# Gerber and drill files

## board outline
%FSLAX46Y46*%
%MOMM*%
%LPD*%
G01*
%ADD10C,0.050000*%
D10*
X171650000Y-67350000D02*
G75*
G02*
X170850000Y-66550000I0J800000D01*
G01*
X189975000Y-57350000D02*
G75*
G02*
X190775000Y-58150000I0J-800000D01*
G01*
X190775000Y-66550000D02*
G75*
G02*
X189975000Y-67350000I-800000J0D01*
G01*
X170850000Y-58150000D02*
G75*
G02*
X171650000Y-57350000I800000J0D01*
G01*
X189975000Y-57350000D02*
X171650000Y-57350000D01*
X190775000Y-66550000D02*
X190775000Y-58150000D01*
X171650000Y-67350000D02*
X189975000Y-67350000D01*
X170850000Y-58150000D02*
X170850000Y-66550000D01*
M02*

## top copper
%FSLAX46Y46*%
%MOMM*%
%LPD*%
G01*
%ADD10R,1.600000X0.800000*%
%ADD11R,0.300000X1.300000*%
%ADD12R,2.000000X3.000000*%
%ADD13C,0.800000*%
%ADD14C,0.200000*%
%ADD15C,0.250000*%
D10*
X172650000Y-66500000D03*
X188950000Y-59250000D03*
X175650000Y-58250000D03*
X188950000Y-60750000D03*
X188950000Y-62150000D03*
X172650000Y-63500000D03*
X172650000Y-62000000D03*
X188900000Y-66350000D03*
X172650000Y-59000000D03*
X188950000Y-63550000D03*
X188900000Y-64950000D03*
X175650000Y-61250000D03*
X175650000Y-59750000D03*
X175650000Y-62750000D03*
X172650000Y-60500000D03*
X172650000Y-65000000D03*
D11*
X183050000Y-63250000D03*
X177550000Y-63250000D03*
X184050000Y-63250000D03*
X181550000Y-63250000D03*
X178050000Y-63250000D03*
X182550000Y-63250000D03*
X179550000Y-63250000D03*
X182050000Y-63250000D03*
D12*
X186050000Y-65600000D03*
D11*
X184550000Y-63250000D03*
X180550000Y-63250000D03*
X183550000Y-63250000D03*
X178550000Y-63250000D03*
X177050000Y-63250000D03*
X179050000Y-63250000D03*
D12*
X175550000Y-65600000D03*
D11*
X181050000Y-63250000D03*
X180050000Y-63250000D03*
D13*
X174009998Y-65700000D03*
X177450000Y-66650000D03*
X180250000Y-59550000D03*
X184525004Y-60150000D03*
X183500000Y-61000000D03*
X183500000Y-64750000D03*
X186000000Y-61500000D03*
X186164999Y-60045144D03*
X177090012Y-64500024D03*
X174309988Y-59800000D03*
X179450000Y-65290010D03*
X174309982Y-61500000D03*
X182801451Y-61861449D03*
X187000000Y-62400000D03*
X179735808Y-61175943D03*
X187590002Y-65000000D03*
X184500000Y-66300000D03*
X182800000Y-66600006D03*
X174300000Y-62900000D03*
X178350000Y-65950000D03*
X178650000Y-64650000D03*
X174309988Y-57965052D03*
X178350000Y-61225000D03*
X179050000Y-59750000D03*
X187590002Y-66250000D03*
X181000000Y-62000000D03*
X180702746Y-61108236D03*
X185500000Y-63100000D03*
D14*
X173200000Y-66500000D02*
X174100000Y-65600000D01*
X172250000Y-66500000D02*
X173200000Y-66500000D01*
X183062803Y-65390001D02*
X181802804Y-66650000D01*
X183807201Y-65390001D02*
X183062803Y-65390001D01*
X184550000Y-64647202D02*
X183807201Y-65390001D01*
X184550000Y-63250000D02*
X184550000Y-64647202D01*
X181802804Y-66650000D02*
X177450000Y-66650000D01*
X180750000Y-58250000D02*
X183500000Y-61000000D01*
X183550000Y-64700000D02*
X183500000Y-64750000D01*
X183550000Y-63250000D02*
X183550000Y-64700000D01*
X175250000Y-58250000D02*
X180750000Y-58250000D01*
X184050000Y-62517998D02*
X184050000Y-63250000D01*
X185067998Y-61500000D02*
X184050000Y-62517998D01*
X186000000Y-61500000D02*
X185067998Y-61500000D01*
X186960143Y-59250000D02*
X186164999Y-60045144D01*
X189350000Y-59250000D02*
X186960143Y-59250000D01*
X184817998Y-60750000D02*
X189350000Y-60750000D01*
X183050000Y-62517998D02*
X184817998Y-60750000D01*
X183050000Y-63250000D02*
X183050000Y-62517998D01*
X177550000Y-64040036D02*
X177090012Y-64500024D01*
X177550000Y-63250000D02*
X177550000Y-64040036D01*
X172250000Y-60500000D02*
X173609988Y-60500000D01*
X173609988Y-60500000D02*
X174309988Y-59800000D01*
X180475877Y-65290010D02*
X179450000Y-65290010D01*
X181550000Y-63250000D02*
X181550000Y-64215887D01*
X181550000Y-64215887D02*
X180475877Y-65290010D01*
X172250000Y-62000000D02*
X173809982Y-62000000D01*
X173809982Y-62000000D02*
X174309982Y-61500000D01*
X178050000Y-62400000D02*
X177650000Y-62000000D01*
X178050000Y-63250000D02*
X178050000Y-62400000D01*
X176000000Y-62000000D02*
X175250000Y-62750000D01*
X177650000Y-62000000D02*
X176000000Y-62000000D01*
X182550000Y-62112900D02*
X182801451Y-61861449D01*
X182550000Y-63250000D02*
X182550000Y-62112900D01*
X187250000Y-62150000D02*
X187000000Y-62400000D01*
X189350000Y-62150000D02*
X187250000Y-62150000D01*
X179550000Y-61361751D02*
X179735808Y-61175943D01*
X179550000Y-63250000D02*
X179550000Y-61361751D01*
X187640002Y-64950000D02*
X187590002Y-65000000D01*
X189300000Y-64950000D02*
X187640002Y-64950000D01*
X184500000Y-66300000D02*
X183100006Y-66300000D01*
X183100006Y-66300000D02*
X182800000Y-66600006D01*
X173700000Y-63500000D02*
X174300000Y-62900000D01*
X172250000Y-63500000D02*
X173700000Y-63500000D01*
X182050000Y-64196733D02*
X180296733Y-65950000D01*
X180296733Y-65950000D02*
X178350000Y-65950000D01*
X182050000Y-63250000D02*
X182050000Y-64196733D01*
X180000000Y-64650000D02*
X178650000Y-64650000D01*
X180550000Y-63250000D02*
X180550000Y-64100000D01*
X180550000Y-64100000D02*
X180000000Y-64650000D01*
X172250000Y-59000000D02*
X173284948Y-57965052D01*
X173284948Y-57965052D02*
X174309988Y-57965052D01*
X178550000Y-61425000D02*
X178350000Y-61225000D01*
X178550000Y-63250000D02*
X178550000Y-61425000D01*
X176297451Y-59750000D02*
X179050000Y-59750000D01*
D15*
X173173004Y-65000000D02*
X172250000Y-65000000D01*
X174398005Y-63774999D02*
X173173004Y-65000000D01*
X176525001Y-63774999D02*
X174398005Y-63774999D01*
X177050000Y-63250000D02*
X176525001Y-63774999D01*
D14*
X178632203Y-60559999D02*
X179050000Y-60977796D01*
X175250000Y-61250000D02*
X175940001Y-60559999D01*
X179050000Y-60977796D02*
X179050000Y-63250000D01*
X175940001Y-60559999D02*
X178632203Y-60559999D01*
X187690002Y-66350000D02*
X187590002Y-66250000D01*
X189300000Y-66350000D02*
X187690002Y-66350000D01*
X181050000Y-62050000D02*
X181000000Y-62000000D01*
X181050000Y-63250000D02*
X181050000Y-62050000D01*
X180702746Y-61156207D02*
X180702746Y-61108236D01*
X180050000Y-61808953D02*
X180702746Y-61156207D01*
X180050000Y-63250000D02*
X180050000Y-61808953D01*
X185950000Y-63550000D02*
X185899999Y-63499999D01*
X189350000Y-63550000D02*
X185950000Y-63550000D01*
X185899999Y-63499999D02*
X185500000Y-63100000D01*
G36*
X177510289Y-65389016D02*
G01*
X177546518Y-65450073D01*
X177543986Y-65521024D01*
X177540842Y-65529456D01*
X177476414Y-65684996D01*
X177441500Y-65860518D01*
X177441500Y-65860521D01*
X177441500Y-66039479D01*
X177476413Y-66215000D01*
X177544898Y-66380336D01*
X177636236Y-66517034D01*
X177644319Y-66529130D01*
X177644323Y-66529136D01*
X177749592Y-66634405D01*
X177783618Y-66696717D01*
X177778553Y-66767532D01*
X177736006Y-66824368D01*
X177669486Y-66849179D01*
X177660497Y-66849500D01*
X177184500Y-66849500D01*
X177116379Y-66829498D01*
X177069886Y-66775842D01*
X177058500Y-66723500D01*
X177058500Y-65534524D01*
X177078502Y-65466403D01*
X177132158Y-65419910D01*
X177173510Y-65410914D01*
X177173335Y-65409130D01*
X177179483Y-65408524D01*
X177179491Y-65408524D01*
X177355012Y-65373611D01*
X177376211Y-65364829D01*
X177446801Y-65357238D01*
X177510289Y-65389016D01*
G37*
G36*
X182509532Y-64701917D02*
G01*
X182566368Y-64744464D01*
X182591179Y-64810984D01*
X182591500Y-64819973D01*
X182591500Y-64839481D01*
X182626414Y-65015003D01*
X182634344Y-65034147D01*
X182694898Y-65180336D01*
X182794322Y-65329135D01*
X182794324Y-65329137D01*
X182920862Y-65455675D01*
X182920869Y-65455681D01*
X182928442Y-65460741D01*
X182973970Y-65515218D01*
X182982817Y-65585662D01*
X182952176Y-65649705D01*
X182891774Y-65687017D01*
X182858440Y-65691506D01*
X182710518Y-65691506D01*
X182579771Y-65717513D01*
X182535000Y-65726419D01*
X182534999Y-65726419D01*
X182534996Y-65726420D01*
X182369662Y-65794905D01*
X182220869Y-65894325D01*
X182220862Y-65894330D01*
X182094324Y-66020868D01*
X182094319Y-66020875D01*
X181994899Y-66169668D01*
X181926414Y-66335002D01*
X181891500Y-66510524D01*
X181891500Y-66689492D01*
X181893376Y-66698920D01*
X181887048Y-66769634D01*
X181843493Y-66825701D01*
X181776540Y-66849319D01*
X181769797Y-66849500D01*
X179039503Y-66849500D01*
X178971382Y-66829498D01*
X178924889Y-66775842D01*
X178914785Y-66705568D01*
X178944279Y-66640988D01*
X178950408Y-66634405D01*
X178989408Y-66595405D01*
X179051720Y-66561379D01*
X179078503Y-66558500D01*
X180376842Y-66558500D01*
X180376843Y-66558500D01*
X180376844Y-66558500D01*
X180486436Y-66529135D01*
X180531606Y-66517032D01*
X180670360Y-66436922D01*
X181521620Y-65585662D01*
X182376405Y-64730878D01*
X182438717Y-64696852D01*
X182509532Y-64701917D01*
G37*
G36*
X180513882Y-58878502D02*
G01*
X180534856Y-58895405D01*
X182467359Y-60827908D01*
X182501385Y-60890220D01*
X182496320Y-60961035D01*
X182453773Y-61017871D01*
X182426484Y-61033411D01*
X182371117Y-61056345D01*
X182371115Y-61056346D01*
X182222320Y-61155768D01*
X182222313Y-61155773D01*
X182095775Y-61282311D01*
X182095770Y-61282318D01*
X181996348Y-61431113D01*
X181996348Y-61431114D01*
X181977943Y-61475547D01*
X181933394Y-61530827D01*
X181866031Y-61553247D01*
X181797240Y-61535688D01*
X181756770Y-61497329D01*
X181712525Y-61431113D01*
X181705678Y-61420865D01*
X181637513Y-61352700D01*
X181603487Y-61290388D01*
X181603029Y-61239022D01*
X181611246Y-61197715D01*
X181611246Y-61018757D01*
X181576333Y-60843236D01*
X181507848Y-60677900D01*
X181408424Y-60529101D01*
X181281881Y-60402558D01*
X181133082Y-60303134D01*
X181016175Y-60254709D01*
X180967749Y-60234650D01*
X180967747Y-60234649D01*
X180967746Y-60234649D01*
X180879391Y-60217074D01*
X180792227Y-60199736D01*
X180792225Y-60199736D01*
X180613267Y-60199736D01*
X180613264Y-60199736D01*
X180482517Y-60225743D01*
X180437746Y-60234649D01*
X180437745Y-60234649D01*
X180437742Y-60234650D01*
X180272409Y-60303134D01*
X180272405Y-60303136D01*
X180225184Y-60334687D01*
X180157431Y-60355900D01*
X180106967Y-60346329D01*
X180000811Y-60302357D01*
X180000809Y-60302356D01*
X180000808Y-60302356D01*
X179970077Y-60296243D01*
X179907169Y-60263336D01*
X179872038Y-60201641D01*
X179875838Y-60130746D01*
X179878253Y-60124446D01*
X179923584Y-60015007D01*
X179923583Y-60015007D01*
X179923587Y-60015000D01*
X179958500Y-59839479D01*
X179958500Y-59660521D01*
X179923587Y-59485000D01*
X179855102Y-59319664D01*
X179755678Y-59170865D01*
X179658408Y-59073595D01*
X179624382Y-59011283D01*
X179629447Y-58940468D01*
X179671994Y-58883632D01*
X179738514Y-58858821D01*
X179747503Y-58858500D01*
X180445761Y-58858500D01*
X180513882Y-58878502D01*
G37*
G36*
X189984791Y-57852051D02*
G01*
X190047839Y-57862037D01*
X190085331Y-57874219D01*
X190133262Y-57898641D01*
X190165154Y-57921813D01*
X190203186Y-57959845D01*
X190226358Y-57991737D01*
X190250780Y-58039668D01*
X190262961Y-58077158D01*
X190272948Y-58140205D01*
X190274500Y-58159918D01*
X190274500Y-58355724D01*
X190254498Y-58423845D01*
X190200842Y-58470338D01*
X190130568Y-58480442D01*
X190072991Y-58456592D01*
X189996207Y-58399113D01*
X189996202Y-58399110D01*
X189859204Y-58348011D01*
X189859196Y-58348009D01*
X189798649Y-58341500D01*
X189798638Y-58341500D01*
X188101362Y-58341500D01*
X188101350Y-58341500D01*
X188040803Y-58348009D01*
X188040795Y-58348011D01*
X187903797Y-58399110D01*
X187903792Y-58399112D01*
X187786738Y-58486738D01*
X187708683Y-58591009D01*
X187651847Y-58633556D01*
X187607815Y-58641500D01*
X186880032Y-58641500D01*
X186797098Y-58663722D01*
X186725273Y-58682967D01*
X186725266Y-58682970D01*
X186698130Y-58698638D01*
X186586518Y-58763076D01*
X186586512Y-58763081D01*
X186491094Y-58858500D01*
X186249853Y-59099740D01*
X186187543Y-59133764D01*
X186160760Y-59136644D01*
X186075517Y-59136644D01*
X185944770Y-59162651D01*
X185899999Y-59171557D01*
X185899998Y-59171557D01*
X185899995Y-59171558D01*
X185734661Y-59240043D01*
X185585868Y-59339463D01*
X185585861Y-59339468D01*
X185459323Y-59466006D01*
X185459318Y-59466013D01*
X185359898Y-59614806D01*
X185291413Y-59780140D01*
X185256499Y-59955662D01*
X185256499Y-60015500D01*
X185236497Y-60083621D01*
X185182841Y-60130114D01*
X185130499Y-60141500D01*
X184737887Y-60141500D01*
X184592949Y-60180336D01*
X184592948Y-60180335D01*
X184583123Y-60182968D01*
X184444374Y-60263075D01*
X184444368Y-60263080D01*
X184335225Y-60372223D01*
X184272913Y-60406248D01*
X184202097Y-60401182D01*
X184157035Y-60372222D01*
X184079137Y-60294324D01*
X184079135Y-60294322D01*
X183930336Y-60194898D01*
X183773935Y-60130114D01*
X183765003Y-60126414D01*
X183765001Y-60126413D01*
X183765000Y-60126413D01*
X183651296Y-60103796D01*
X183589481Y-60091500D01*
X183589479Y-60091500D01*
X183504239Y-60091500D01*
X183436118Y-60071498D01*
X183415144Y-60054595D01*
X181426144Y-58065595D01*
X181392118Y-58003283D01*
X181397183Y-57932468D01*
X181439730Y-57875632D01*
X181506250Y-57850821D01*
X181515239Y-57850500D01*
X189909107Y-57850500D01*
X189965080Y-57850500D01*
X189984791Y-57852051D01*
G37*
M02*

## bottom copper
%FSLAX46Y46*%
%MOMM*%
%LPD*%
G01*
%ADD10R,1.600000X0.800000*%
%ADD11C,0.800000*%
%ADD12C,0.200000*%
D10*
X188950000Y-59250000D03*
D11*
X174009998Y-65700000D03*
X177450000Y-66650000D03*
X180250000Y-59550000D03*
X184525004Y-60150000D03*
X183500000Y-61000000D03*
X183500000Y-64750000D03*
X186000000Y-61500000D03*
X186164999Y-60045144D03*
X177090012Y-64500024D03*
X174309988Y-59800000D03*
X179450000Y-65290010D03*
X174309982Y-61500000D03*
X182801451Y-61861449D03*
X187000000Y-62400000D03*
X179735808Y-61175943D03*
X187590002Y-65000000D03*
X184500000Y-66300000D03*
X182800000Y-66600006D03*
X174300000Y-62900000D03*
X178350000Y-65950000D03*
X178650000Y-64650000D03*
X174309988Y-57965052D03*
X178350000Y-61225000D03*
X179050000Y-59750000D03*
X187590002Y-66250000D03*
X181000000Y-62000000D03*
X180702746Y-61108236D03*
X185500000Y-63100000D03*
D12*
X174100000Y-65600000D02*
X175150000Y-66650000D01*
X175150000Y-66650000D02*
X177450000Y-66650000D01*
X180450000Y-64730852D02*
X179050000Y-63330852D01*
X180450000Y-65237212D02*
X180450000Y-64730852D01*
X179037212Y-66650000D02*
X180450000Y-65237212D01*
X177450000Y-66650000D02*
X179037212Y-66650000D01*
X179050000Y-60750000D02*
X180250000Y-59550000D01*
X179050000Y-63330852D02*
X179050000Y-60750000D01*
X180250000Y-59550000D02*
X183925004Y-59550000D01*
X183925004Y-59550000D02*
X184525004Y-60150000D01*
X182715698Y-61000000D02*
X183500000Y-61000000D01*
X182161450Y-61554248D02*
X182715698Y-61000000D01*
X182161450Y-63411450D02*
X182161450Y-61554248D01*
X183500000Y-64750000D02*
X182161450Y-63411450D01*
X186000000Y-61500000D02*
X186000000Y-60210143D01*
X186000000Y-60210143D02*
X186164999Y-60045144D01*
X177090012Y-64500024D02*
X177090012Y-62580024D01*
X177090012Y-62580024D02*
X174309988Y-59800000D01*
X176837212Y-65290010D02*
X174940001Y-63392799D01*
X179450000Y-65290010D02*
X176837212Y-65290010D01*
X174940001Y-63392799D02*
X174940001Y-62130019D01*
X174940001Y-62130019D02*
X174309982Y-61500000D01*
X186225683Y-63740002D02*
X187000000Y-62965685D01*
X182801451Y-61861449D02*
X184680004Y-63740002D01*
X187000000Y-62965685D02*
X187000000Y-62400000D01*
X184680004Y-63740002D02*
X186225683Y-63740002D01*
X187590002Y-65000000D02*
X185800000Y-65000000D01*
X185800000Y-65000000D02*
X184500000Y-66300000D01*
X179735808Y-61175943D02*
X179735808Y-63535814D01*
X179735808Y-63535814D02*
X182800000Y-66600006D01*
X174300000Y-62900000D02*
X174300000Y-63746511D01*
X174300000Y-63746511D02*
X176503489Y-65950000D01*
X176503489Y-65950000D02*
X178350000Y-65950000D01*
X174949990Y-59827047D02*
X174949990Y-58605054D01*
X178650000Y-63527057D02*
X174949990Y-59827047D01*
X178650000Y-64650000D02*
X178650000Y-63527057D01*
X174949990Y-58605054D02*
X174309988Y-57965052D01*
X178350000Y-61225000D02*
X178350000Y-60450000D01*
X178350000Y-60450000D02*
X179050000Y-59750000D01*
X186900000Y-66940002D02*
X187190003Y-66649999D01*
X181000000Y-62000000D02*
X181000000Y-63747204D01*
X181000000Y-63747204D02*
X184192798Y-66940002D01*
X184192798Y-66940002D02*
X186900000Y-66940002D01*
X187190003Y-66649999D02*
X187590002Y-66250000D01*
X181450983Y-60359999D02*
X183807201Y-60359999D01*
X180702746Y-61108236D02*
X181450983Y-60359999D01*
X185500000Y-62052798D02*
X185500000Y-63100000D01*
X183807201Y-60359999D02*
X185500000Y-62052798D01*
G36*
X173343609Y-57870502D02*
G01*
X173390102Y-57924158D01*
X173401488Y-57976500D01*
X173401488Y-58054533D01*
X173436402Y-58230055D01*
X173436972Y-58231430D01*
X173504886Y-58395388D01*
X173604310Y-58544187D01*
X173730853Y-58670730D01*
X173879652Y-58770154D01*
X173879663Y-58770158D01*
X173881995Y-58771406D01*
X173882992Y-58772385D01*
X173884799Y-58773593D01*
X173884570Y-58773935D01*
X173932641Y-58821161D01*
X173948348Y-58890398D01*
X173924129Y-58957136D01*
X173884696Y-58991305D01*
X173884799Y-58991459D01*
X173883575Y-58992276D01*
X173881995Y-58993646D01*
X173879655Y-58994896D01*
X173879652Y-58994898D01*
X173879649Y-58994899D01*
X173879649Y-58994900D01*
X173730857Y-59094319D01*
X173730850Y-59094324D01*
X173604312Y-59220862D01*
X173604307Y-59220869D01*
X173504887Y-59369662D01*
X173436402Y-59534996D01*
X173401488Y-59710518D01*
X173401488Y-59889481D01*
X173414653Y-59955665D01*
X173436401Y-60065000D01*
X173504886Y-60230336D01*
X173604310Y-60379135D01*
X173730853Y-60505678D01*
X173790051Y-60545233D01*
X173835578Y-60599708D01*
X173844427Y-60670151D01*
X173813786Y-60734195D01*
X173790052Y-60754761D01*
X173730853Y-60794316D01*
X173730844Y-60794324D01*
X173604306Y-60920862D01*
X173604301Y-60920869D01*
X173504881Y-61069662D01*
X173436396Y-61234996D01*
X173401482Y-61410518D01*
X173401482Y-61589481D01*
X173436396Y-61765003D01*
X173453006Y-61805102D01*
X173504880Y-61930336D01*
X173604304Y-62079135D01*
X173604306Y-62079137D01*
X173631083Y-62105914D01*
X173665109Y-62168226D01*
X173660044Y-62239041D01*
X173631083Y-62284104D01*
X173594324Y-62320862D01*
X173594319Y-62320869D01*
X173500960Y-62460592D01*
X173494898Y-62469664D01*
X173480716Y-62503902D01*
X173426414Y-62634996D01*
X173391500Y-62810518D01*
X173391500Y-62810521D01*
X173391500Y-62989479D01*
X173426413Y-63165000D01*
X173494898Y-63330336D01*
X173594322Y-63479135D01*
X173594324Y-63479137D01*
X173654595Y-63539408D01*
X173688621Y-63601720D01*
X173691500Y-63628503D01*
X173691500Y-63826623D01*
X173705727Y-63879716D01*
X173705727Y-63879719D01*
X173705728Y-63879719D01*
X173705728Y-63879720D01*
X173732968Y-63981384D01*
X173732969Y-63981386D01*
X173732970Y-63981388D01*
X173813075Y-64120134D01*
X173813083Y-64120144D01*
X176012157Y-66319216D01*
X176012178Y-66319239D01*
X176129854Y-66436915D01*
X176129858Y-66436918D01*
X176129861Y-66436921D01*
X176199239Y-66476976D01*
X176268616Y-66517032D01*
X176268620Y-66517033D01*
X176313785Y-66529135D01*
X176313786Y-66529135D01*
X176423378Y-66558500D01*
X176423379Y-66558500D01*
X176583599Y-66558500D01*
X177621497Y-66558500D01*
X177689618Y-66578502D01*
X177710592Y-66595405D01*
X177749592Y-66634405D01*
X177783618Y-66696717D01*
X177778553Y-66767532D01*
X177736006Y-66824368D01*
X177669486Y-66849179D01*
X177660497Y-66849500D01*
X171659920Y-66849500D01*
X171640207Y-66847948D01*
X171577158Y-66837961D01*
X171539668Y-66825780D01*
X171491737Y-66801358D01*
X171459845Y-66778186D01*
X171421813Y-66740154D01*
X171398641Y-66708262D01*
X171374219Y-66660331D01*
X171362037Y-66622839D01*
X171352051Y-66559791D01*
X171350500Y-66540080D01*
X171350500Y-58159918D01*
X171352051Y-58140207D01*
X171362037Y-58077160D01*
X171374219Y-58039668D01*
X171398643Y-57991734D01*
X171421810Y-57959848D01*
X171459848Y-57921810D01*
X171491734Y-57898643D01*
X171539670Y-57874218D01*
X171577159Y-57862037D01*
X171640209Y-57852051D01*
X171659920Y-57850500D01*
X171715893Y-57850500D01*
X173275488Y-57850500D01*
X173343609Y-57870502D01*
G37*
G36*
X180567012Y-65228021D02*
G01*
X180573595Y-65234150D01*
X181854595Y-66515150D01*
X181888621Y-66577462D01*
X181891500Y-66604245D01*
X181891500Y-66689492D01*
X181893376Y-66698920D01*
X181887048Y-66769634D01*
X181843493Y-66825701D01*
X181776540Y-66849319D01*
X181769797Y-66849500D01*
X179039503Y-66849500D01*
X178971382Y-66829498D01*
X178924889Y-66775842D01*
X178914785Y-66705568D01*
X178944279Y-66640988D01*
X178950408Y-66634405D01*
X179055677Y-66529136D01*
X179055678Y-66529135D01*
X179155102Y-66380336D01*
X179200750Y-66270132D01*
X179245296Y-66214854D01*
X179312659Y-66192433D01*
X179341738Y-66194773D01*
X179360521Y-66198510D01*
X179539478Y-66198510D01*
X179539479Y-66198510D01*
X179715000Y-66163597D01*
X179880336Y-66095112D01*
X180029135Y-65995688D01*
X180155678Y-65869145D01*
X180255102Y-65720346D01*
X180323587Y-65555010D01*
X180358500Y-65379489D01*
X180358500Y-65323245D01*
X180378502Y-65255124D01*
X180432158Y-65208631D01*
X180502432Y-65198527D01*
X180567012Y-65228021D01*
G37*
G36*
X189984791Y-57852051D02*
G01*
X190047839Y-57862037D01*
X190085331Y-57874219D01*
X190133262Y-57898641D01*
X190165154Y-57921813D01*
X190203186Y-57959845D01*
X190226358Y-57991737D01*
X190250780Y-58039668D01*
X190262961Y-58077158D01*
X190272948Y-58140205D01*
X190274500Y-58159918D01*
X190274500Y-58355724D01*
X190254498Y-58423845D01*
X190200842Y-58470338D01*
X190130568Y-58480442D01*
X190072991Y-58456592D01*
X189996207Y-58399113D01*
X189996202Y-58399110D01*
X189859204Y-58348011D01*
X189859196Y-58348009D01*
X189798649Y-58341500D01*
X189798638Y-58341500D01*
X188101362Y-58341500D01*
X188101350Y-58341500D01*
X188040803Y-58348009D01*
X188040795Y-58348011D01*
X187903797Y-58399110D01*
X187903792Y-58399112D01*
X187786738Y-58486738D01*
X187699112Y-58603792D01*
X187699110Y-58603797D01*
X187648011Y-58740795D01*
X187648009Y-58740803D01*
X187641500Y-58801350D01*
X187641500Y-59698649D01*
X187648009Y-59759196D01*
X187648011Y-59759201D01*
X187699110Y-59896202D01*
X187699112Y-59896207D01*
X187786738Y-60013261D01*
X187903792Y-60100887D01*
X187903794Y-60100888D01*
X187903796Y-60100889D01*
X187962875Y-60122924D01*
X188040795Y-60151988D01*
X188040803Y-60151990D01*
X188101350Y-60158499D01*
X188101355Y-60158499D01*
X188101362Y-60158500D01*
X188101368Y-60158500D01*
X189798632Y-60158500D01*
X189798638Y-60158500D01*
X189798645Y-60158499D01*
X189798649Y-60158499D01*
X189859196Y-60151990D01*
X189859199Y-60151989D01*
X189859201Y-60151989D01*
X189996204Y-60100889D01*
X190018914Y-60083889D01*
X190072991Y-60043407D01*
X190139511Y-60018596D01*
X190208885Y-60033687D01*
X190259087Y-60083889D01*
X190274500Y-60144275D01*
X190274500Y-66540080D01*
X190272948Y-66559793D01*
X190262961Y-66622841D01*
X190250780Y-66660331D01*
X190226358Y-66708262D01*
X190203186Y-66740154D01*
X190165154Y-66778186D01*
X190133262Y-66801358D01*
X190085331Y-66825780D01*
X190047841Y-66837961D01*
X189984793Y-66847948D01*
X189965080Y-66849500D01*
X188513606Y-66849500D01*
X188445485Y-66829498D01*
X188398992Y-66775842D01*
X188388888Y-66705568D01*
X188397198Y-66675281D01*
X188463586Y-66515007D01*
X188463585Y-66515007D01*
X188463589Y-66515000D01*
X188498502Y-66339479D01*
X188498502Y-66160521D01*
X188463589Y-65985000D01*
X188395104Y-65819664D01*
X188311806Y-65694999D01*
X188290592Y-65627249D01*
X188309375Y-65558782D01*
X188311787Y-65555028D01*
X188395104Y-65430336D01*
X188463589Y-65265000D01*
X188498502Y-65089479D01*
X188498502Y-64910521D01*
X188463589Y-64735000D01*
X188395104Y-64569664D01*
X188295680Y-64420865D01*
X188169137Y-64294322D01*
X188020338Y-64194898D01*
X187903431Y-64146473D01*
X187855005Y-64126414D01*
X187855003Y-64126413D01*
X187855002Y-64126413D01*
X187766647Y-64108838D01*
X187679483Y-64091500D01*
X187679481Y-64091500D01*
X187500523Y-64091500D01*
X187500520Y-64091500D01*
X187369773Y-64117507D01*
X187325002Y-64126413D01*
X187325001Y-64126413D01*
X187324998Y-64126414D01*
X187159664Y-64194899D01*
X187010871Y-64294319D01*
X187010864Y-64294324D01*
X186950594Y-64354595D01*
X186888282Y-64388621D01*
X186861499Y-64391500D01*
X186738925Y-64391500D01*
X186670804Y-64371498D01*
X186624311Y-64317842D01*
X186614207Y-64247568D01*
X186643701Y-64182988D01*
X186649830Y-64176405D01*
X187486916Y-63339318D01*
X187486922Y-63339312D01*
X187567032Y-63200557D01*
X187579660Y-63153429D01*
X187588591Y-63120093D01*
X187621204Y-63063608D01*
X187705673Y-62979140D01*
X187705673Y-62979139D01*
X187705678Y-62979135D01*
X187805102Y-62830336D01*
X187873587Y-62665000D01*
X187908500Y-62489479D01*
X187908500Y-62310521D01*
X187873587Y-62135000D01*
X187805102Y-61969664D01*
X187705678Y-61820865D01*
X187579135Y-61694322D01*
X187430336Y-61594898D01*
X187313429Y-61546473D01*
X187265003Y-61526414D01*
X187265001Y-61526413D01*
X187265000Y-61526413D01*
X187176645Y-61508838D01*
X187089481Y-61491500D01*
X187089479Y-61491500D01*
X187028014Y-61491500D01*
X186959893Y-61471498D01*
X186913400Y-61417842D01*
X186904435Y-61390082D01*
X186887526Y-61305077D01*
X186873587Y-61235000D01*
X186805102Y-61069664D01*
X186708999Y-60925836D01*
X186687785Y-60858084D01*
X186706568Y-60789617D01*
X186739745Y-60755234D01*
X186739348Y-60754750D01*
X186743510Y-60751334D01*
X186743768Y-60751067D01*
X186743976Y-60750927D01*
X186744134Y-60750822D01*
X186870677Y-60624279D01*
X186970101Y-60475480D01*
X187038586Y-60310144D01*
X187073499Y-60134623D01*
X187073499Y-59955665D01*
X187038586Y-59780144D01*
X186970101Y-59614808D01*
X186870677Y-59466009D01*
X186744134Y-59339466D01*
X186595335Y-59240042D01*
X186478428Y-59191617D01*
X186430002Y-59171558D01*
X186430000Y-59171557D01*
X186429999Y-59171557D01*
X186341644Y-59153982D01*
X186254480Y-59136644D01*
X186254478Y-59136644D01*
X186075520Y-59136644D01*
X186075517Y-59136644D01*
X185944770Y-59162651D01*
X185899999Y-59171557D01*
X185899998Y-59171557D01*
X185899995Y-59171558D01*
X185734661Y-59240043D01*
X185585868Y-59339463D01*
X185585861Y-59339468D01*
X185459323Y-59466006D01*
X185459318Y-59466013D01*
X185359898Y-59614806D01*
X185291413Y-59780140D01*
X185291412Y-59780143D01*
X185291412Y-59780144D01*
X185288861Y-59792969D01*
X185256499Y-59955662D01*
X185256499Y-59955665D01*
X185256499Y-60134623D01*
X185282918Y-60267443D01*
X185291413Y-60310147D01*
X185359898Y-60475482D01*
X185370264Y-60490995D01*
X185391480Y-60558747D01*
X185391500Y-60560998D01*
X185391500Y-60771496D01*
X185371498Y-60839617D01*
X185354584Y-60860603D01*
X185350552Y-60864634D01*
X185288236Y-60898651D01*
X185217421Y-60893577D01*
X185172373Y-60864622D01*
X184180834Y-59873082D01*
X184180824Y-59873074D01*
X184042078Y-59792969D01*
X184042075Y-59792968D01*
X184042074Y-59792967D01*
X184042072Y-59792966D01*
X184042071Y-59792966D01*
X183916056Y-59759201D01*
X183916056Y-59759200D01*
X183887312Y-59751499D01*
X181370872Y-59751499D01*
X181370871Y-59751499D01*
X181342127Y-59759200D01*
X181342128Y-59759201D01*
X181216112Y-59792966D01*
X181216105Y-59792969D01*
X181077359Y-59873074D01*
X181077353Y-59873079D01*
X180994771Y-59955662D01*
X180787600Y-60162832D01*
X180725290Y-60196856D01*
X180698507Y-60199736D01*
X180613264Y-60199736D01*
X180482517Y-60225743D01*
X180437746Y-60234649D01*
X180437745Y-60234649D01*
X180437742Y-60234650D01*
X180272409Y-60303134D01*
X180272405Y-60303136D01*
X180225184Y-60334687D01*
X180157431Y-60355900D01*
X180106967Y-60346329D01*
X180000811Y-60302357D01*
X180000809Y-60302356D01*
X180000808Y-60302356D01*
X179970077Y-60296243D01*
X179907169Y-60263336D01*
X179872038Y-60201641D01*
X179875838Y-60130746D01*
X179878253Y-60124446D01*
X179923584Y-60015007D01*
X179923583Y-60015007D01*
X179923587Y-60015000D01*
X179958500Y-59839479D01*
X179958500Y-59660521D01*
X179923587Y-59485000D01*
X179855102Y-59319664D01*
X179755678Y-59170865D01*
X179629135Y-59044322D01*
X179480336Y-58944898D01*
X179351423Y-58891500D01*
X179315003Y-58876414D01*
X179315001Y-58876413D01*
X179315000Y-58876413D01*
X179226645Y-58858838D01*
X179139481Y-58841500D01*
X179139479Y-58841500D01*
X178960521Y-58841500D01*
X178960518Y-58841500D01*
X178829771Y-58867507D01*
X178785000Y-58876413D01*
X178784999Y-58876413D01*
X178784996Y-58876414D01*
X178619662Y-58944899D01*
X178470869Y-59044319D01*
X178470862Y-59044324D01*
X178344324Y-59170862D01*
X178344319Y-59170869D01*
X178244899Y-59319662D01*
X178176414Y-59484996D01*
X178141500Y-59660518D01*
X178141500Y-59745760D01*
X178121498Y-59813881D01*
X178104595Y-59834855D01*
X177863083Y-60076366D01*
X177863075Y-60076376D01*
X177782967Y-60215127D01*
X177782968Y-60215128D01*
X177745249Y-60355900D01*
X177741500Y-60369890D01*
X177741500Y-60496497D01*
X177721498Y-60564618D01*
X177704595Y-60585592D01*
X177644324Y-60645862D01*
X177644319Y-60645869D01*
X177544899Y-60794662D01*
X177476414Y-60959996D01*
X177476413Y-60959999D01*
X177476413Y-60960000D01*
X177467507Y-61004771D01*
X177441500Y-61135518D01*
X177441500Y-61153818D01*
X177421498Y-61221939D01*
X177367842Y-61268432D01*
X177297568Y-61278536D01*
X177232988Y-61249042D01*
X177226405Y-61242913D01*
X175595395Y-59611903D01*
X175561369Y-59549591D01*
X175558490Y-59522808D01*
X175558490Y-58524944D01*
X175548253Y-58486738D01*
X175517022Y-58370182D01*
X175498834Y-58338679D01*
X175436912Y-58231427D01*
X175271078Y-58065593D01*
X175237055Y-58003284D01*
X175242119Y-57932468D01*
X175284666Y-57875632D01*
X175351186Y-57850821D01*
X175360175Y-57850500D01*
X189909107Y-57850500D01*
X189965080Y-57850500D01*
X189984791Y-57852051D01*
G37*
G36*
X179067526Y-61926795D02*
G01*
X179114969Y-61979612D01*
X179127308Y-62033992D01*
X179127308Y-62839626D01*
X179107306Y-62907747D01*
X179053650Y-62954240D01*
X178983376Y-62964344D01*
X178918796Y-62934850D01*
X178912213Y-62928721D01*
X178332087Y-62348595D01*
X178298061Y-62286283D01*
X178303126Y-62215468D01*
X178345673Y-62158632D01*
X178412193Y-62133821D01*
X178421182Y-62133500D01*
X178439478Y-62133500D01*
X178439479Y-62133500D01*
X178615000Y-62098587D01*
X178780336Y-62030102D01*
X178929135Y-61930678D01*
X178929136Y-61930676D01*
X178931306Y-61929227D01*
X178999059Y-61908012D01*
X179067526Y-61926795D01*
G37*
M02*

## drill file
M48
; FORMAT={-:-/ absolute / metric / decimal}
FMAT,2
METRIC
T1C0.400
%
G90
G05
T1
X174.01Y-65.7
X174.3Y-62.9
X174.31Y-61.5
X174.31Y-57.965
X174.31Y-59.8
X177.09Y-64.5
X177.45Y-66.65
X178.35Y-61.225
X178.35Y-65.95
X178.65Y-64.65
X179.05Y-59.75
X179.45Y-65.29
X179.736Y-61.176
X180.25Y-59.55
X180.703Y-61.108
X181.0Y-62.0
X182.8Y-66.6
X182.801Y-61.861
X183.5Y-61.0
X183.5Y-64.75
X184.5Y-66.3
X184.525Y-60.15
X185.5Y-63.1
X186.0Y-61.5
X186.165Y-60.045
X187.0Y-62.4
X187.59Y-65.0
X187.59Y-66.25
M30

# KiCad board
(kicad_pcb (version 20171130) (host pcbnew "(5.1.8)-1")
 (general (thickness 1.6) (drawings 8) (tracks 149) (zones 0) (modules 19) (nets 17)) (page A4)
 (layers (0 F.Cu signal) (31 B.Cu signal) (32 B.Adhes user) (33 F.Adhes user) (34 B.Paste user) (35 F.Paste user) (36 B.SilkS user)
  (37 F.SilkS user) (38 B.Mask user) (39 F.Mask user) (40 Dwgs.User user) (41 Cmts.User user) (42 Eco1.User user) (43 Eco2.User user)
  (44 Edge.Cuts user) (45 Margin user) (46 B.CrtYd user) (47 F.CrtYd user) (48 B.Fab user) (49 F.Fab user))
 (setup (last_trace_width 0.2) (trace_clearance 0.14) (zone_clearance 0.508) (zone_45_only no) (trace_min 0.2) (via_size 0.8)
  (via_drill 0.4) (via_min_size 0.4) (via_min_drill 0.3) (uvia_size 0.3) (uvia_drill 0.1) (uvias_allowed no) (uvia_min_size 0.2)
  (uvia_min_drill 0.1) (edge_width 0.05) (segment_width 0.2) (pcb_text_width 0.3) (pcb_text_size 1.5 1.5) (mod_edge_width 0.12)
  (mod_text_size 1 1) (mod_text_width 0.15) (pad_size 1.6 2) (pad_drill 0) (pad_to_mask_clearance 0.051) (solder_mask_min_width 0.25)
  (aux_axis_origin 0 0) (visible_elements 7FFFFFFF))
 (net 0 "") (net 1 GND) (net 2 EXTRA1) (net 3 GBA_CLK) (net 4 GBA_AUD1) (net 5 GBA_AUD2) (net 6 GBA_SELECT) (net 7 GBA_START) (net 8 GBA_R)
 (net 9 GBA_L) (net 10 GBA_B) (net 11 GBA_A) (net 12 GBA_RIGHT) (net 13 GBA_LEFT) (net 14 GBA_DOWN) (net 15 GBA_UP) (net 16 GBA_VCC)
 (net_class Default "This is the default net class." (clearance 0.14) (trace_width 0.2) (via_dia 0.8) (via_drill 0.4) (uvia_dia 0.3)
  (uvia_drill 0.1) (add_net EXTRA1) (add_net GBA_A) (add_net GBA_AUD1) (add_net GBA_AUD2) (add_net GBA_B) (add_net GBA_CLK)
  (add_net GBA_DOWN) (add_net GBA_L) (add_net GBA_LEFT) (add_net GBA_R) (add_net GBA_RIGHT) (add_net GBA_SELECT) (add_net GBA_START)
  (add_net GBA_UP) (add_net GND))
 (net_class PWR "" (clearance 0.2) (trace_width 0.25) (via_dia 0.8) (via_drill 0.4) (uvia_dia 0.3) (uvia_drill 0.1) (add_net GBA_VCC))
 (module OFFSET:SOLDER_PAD (layer B.Cu) (at 188.8 59.25 270)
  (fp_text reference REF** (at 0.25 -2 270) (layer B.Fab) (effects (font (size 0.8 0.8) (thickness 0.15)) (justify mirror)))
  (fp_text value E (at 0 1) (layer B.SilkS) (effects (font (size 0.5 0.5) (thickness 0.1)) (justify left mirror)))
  (pad 1 smd rect (at 0 0.25 270) (size 0.8 1.6) (drill (offset 0 -0.4)) (layers B.Cu B.Paste B.Mask)))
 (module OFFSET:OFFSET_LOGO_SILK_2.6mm (layer B.Cu) (at 180.575 62.275 180)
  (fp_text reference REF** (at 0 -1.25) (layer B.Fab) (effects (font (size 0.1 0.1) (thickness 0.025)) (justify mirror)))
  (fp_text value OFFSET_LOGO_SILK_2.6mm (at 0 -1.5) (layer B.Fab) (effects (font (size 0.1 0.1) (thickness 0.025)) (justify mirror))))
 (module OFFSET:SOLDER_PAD (layer F.Cu) (at 172.5 66.5 90)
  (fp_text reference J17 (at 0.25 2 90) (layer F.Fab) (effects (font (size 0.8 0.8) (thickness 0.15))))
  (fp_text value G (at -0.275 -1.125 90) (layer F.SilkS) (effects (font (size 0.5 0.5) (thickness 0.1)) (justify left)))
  (pad 1 smd rect (at 0 -0.25 90) (size 0.8 1.6) (drill (offset 0 0.4)) (layers F.Cu F.Paste F.Mask) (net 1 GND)))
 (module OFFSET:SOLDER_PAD (layer F.Cu) (at 189.1 59.25 270)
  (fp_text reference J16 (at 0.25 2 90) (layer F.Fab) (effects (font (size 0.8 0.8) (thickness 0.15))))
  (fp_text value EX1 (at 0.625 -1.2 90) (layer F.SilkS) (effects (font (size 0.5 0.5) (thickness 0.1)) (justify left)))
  (pad 1 smd rect (at 0 -0.25 270) (size 0.8 1.6) (drill (offset 0 0.4)) (layers F.Cu F.Paste F.Mask) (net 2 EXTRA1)))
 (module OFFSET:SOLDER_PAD (layer F.Cu) (at 175.5 58.25 90)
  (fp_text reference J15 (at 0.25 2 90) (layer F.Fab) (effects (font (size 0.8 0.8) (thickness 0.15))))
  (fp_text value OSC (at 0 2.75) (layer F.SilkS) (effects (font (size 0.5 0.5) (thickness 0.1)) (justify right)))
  (pad 1 smd rect (at 0 -0.25 90) (size 0.8 1.6) (drill (offset 0 0.4)) (layers F.Cu F.Paste F.Mask) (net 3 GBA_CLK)))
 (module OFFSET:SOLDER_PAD (layer F.Cu) (at 189.1 60.75 270)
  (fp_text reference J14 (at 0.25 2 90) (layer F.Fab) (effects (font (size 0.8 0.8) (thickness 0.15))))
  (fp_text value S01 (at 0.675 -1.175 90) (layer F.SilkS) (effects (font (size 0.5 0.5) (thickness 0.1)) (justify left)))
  (pad 1 smd rect (at 0 -0.25 270) (size 0.8 1.6) (drill (offset 0 0.4)) (layers F.Cu F.Paste F.Mask) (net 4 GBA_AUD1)))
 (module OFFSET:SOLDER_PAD (layer F.Cu) (at 189.1 62.15 270)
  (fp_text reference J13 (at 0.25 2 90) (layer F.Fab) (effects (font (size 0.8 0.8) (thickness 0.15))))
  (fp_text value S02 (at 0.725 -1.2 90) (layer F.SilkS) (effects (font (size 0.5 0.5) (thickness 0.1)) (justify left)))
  (pad 1 smd rect (at 0 -0.25 270) (size 0.8 1.6) (drill (offset 0 0.4)) (layers F.Cu F.Paste F.Mask) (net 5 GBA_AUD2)))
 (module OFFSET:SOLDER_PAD (layer F.Cu) (at 172.5 63.5 90)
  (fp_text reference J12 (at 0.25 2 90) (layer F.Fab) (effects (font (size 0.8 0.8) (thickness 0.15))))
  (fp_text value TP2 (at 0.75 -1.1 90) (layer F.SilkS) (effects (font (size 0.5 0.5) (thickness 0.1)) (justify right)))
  (pad 1 smd rect (at 0 -0.25 90) (size 0.8 1.6) (drill (offset 0 0.4)) (layers F.Cu F.Paste F.Mask) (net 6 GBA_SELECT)))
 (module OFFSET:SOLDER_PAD (layer F.Cu) (at 172.5 62 90)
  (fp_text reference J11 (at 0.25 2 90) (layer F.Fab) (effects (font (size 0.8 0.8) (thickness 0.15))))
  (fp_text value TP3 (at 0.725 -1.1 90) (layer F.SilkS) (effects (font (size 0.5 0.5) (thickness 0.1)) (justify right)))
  (pad 1 smd rect (at 0 -0.25 90) (size 0.8 1.6) (drill (offset 0 0.4)) (layers F.Cu F.Paste F.Mask) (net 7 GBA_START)))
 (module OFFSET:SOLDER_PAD (layer F.Cu) (at 189.05 66.35 270)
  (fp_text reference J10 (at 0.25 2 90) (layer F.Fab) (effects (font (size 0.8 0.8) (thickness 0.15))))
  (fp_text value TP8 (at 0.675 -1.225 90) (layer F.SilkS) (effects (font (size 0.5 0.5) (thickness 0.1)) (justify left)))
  (pad 1 smd rect (at 0 -0.25 270) (size 0.8 1.6) (drill (offset 0 0.4)) (layers F.Cu F.Paste F.Mask) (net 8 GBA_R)))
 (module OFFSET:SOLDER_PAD (layer F.Cu) (at 172.5 59 90)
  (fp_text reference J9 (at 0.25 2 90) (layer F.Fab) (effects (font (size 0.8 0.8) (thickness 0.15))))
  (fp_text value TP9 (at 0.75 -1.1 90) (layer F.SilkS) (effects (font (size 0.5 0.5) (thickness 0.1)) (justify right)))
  (pad 1 smd rect (at 0 -0.25 90) (size 0.8 1.6) (drill (offset 0 0.4)) (layers F.Cu F.Paste F.Mask) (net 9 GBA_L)))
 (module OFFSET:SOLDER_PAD (layer F.Cu) (at 189.1 63.55 270)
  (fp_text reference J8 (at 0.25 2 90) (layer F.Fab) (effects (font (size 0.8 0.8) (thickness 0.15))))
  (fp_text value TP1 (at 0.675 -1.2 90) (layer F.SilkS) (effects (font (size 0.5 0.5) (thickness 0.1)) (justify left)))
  (pad 1 smd rect (at 0 -0.25 270) (size 0.8 1.6) (drill (offset 0 0.4)) (layers F.Cu F.Paste F.Mask) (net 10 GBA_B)))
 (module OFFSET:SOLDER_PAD (layer F.Cu) (at 189.05 64.95 270)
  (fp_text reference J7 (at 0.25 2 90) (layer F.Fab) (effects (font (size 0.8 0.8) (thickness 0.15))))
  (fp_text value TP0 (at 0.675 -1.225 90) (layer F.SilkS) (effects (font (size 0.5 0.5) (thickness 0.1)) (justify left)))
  (pad 1 smd rect (at 0 -0.25 270) (size 0.8 1.6) (drill (offset 0 0.4)) (layers F.Cu F.Paste F.Mask) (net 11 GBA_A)))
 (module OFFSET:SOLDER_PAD (layer F.Cu) (at 175.5 61.25 90)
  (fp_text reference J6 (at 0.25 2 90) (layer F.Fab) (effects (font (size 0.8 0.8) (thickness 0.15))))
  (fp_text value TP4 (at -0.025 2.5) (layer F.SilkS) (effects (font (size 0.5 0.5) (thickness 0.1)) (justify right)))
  (pad 1 smd rect (at 0 -0.25 90) (size 0.8 1.6) (drill (offset 0 0.4)) (layers F.Cu F.Paste F.Mask) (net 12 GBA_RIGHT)))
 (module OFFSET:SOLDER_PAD (layer F.Cu) (at 175.5 59.75 90)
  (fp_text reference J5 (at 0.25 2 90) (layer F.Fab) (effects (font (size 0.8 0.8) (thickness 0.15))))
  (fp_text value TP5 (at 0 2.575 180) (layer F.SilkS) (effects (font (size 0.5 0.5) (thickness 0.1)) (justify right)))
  (pad 1 smd rect (at 0 -0.25 90) (size 0.8 1.6) (drill (offset 0 0.4)) (layers F.Cu F.Paste F.Mask) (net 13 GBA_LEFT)))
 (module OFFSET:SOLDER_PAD (layer F.Cu) (at 175.5 62.75 90)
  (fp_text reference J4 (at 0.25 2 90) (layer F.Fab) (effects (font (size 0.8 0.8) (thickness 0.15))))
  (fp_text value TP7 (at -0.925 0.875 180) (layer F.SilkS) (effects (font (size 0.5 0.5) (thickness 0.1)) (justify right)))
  (pad 1 smd rect (at 0 -0.25 90) (size 0.8 1.6) (drill (offset 0 0.4)) (layers F.Cu F.Paste F.Mask) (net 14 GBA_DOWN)))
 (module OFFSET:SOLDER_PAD (layer F.Cu) (at 172.5 60.5 90)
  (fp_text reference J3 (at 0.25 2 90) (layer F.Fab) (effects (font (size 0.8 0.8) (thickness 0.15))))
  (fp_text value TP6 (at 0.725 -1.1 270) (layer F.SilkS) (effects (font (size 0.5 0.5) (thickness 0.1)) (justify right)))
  (pad 1 smd rect (at 0 -0.25 90) (size 0.8 1.6) (drill (offset 0 0.4)) (layers F.Cu F.Paste F.Mask) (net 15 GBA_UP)))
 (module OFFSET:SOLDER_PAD (layer F.Cu) (at 172.5 65 90)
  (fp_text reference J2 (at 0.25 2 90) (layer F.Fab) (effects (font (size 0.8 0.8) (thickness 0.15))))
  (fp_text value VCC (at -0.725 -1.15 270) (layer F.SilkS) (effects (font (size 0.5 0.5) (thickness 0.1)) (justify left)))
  (pad 1 smd rect (at 0 -0.25 90) (size 0.8 1.6) (drill (offset 0 0.4)) (layers F.Cu F.Paste F.Mask) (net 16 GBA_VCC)))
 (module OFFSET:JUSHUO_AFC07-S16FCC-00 (layer F.Cu) (at 180.8 65)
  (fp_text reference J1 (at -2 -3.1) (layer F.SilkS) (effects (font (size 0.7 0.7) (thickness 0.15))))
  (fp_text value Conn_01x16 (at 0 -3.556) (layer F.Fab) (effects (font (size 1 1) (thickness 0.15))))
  (pad 13 smd rect (at 2.25 -1.75) (size 0.3 1.3) (layers F.Cu F.Paste F.Mask) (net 4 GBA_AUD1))
  (pad 2 smd rect (at -3.25 -1.75) (size 0.3 1.3) (layers F.Cu F.Paste F.Mask) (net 15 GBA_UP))
  (pad 15 smd rect (at 3.25 -1.75) (size 0.3 1.3) (layers F.Cu F.Paste F.Mask) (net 2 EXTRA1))
  (pad 10 smd rect (at 0.75 -1.75) (size 0.3 1.3) (layers F.Cu F.Paste F.Mask) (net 7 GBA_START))
  (pad 3 smd rect (at -2.75 -1.75) (size 0.3 1.3) (layers F.Cu F.Paste F.Mask) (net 14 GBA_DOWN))
  (pad 12 smd rect (at 1.75 -1.75) (size 0.3 1.3) (layers F.Cu F.Paste F.Mask) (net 5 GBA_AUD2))
  (pad 6 smd rect (at -1.25 -1.75) (size 0.3 1.3) (layers F.Cu F.Paste F.Mask) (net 11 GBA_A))
  (pad 11 smd rect (at 1.25 -1.75) (size 0.3 1.3) (layers F.Cu F.Paste F.Mask) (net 6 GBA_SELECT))
  (pad "" smd rect (at 5.25 0.6) (size 2 3) (layers F.Cu F.Paste F.Mask))
  (pad 16 smd rect (at 3.75 -1.75) (size 0.3 1.3) (layers F.Cu F.Paste F.Mask) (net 1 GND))
  (pad 8 smd rect (at -0.25 -1.75) (size 0.3 1.3) (layers F.Cu F.Paste F.Mask) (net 9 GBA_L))
  (pad 14 smd rect (at 2.75 -1.75) (size 0.3 1.3) (layers F.Cu F.Paste F.Mask) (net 3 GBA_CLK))
  (pad 4 smd rect (at -2.25 -1.75) (size 0.3 1.3) (layers F.Cu F.Paste F.Mask) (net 13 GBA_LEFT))
  (pad 1 smd rect (at -3.75 -1.75) (size 0.3 1.3) (layers F.Cu F.Paste F.Mask) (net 16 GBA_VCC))
  (pad 5 smd rect (at -1.75 -1.75) (size 0.3 1.3) (layers F.Cu F.Paste F.Mask) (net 12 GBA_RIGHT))
  (pad "" smd rect (at -5.25 0.6) (size 2 3) (layers F.Cu F.Paste F.Mask))
  (pad 9 smd rect (at 0.25 -1.75) (size 0.3 1.3) (layers F.Cu F.Paste F.Mask) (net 8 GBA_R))
  (pad 7 smd rect (at -0.75 -1.75) (size 0.3 1.3) (layers F.Cu F.Paste F.Mask) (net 10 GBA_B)))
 (gr_arc (start 171.65 66.55) (end 171.65 67.35) (angle 90) (layer Edge.Cuts) (width 0.05))
 (gr_arc (start 189.975 58.15) (end 190.775 58.15) (angle -90) (layer Edge.Cuts) (width 0.05))
 (gr_arc (start 189.975 66.55) (end 189.975 67.35) (angle -90) (layer Edge.Cuts) (width 0.05))
 (gr_arc (start 171.65 58.15) (end 171.65 57.35) (angle -90) (layer Edge.Cuts) (width 0.05))
 (gr_line (start 189.975 57.35) (end 171.65 57.35) (layer Edge.Cuts) (width 0.05))
 (gr_line (start 190.775 66.55) (end 190.775 58.15) (layer Edge.Cuts) (width 0.05))
 (gr_line (start 171.65 67.35) (end 189.975 67.35) (layer Edge.Cuts) (width 0.05))
 (gr_line (start 170.85 58.15) (end 170.85 66.55) (layer Edge.Cuts) (width 0.05))
 (via (at 174.009998 65.7) (size 0.8) (drill 0.4) (layers F.Cu B.Cu) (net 1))
 (segment (start 173.2 66.5) (end 174.1 65.6) (width 0.2) (layer F.Cu) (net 1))
 (segment (start 172.25 66.5) (end 173.2 66.5) (width 0.2) (layer F.Cu) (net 1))
 (segment (start 183.062803 65.390001) (end 181.802804 66.65) (width 0.2) (layer F.Cu) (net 1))
 (segment (start 183.807201 65.390001) (end 183.062803 65.390001) (width 0.2) (layer F.Cu) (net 1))
 (segment (start 184.55 64.647202) (end 183.807201 65.390001) (width 0.2) (layer F.Cu) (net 1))
 (segment (start 184.55 63.25) (end 184.55 64.647202) (width 0.2) (layer F.Cu) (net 1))
 (segment (start 181.802804 66.65) (end 177.45 66.65) (width 0.2) (layer F.Cu) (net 1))
 (segment (start 174.1 65.6) (end 175.15 66.65) (width 0.2) (layer B.Cu) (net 1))
 (segment (start 175.15 66.65) (end 177.45 66.65) (width 0.2) (layer B.Cu) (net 1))
 (via (at 177.45 66.65) (size 0.8) (drill 0.4) (layers F.Cu B.Cu) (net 1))
 (segment (start 180.45 64.730852) (end 179.05 63.330852) (width 0.2) (layer B.Cu) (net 1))
 (segment (start 180.45 65.237212) (end 180.45 64.730852) (width 0.2) (layer B.Cu) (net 1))
 (segment (start 179.037212 66.65) (end 180.45 65.237212) (width 0.2) (layer B.Cu) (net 1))
 (segment (start 177.45 66.65) (end 179.037212 66.65) (width 0.2) (layer B.Cu) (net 1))
 (via (at 180.25 59.55) (size 0.8) (drill 0.4) (layers F.Cu B.Cu) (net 1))
 (segment (start 179.05 60.75) (end 180.25 59.55) (width 0.2) (layer B.Cu) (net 1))
 (segment (start 179.05 63.330852) (end 179.05 60.75) (width 0.2) (layer B.Cu) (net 1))
 (via (at 184.525004 60.15) (size 0.8) (drill 0.4) (layers F.Cu B.Cu) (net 1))
 (segment (start 180.25 59.55) (end 183.925004 59.55) (width 0.2) (layer B.Cu) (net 1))
 (segment (start 183.925004 59.55) (end 184.525004 60.15) (width 0.2) (layer B.Cu) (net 1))
 (via (at 183.5 61) (size 0.8) (drill 0.4) (layers F.Cu B.Cu) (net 3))
 (segment (start 180.75 58.25) (end 183.5 61) (width 0.2) (layer F.Cu) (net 3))
 (via (at 183.5 64.75) (size 0.8) (drill 0.4) (layers F.Cu B.Cu) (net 3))
 (segment (start 183.55 64.7) (end 183.5 64.75) (width 0.2) (layer F.Cu) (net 3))
 (segment (start 183.55 63.25) (end 183.55 64.7) (width 0.2) (layer F.Cu) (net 3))
 (segment (start 182.715698 61) (end 183.5 61) (width 0.2) (layer B.Cu) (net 3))
 (segment (start 182.16145 61.554248) (end 182.715698 61) (width 0.2) (layer B.Cu) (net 3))
 (segment (start 182.16145 63.41145) (end 182.16145 61.554248) (width 0.2) (layer B.Cu) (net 3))
 (segment (start 183.5 64.75) (end 182.16145 63.41145) (width 0.2) (layer B.Cu) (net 3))
 (segment (start 175.25 58.25) (end 180.75 58.25) (width 0.2) (layer F.Cu) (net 3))
 (via (at 186 61.5) (size 0.8) (drill 0.4) (layers F.Cu B.Cu) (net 2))
 (segment (start 184.05 62.517998) (end 184.05 63.25) (width 0.2) (layer F.Cu) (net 2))
 (segment (start 185.067998 61.5) (end 184.05 62.517998) (width 0.2) (layer F.Cu) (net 2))
 (segment (start 186 61.5) (end 185.067998 61.5) (width 0.2) (layer F.Cu) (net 2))
 (segment (start 186.960143 59.25) (end 186.164999 60.045144) (width 0.2) (layer F.Cu) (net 2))
 (via (at 186.164999 60.045144) (size 0.8) (drill 0.4) (layers F.Cu B.Cu) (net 2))
 (segment (start 189.35 59.25) (end 186.960143 59.25) (width 0.2) (layer F.Cu) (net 2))
 (segment (start 186 61.5) (end 186 60.210143) (width 0.2) (layer B.Cu) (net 2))
 (segment (start 186 60.210143) (end 186.164999 60.045144) (width 0.2) (layer B.Cu) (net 2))
 (segment (start 184.817998 60.75) (end 189.35 60.75) (width 0.2) (layer F.Cu) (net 4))
 (segment (start 183.05 62.517998) (end 184.817998 60.75) (width 0.2) (layer F.Cu) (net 4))
 (segment (start 183.05 63.25) (end 183.05 62.517998) (width 0.2) (layer F.Cu) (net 4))
 (via (at 177.090012 64.500024) (size 0.8) (drill 0.4) (layers F.Cu B.Cu) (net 15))
 (segment (start 177.55 64.040036) (end 177.090012 64.500024) (width 0.2) (layer F.Cu) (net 15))
 (segment (start 177.55 63.25) (end 177.55 64.040036) (width 0.2) (layer F.Cu) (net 15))
 (via (at 174.309988 59.8) (size 0.8) (drill 0.4) (layers F.Cu B.Cu) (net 15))
 (segment (start 172.25 60.5) (end 173.609988 60.5) (width 0.2) (layer F.Cu) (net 15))
 (segment (start 173.609988 60.5) (end 174.309988 59.8) (width 0.2) (layer F.Cu) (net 15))
 (segment (start 177.090012 64.500024) (end 177.090012 62.580024) (width 0.2) (layer B.Cu) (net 15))
 (segment (start 177.090012 62.580024) (end 174.309988 59.8) (width 0.2) (layer B.Cu) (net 15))
 (via (at 179.45 65.29001) (size 0.8) (drill 0.4) (layers F.Cu B.Cu) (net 7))
 (segment (start 180.475877 65.29001) (end 179.45 65.29001) (width 0.2) (layer F.Cu) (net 7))
 (segment (start 181.55 63.25) (end 181.55 64.215887) (width 0.2) (layer F.Cu) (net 7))
 (segment (start 181.55 64.215887) (end 180.475877 65.29001) (width 0.2) (layer F.Cu) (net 7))
 (via (at 174.309982 61.5) (size 0.8) (drill 0.4) (layers F.Cu B.Cu) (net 7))
 (segment (start 176.837212 65.29001) (end 174.940001 63.392799) (width 0.2) (layer B.Cu) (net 7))
 (segment (start 172.25 62) (end 173.809982 62) (width 0.2) (layer F.Cu) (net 7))
 (segment (start 173.809982 62) (end 174.309982 61.5) (width 0.2) (layer F.Cu) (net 7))
 (segment (start 179.45 65.29001) (end 176.837212 65.29001) (width 0.2) (layer B.Cu) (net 7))
 (segment (start 174.940001 63.392799) (end 174.940001 62.130019) (width 0.2) (layer B.Cu) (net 7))
 (segment (start 174.940001 62.130019) (end 174.309982 61.5) (width 0.2) (layer B.Cu) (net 7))
 (segment (start 178.05 62.4) (end 177.65 62) (width 0.2) (layer F.Cu) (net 14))
 (segment (start 178.05 63.25) (end 178.05 62.4) (width 0.2) (layer F.Cu) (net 14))
 (segment (start 176 62) (end 175.25 62.75) (width 0.2) (layer F.Cu) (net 14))
 (segment (start 177.65 62) (end 176 62) (width 0.2) (layer F.Cu) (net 14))
 (segment (start 182.55 62.1129) (end 182.801451 61.861449) (width 0.2) (layer F.Cu) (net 5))
 (via (at 182.801451 61.861449) (size 0.8) (drill 0.4) (layers F.Cu B.Cu) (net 5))
 (segment (start 182.55 63.25) (end 182.55 62.1129) (width 0.2) (layer F.Cu) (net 5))
 (segment (start 187.25 62.15) (end 187 62.4) (width 0.2) (layer F.Cu) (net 5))
 (segment (start 189.35 62.15) (end 187.25 62.15) (width 0.2) (layer F.Cu) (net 5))
 (via (at 187 62.4) (size 0.8) (drill 0.4) (layers F.Cu B.Cu) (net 5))
 (segment (start 186.225683 63.740002) (end 187 62.965685) (width 0.2) (layer B.Cu) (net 5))
 (segment (start 182.801451 61.861449) (end 184.680004 63.740002) (width 0.2) (layer B.Cu) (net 5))
 (segment (start 187 62.965685) (end 187 62.4) (width 0.2) (layer B.Cu) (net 5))
 (segment (start 184.680004 63.740002) (end 186.225683 63.740002) (width 0.2) (layer B.Cu) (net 5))
 (via (at 179.735808 61.175943) (size 0.8) (drill 0.4) (layers F.Cu B.Cu) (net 11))
 (segment (start 179.55 61.361751) (end 179.735808 61.175943) (width 0.2) (layer F.Cu) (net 11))
 (segment (start 179.55 63.25) (end 179.55 61.361751) (width 0.2) (layer F.Cu) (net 11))
 (via (at 187.590002 65) (size 0.8) (drill 0.4) (layers F.Cu B.Cu) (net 11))
 (segment (start 187.640002 64.95) (end 187.590002 65) (width 0.2) (layer F.Cu) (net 11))
 (segment (start 189.3 64.95) (end 187.640002 64.95) (width 0.2) (layer F.Cu) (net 11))
 (via (at 184.5 66.3) (size 0.8) (drill 0.4) (layers F.Cu B.Cu) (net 11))
 (segment (start 187.590002 65) (end 185.8 65) (width 0.2) (layer B.Cu) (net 11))
 (segment (start 185.8 65) (end 184.5 66.3) (width 0.2) (layer B.Cu) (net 11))
 (via (at 182.8 66.600006) (size 0.8) (drill 0.4) (layers F.Cu B.Cu) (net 11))
 (segment (start 184.5 66.3) (end 183.100006 66.3) (width 0.2) (layer F.Cu) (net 11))
 (segment (start 179.735808 61.175943) (end 179.735808 63.535814) (width 0.2) (layer B.Cu) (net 11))
 (segment (start 183.100006 66.3) (end 182.8 66.600006) (width 0.2) (layer F.Cu) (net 11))
 (segment (start 179.735808 63.535814) (end 182.8 66.600006) (width 0.2) (layer B.Cu) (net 11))
 (segment (start 173.7 63.5) (end 174.3 62.9) (width 0.2) (layer F.Cu) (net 6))
 (segment (start 172.25 63.5) (end 173.7 63.5) (width 0.2) (layer F.Cu) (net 6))
 (via (at 174.3 62.9) (size 0.8) (drill 0.4) (layers F.Cu B.Cu) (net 6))
 (via (at 178.35 65.95) (size 0.8) (drill 0.4) (layers F.Cu B.Cu) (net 6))
 (segment (start 182.05 64.196733) (end 180.296733 65.95) (width 0.2) (layer F.Cu) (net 6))
 (segment (start 174.3 62.9) (end 174.3 63.746511) (width 0.2) (layer B.Cu) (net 6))
 (segment (start 174.3 63.746511) (end 176.503489 65.95) (width 0.2) (layer B.Cu) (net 6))
 (segment (start 180.296733 65.95) (end 178.35 65.95) (width 0.2) (layer F.Cu) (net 6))
 (segment (start 176.503489 65.95) (end 178.35 65.95) (width 0.2) (layer B.Cu) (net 6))
 (segment (start 182.05 63.25) (end 182.05 64.196733) (width 0.2) (layer F.Cu) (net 6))
 (segment (start 180 64.65) (end 178.65 64.65) (width 0.2) (layer F.Cu) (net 9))
 (via (at 178.65 64.65) (size 0.8) (drill 0.4) (layers F.Cu B.Cu) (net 9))
 (segment (start 180.55 63.25) (end 180.55 64.1) (width 0.2) (layer F.Cu) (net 9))
 (segment (start 180.55 64.1) (end 180 64.65) (width 0.2) (layer F.Cu) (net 9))
 (via (at 174.309988 57.965052) (size 0.8) (drill 0.4) (layers F.Cu B.Cu) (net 9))
 (segment (start 174.94999 59.827047) (end 174.94999 58.605054) (width 0.2) (layer B.Cu) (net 9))
 (segment (start 172.25 59) (end 173.284948 57.965052) (width 0.2) (layer F.Cu) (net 9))
 (segment (start 178.65 63.527057) (end 174.94999 59.827047) (width 0.2) (layer B.Cu) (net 9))
 (segment (start 173.284948 57.965052) (end 174.309988 57.965052) (width 0.2) (layer F.Cu) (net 9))
 (segment (start 178.65 64.65) (end 178.65 63.527057) (width 0.2) (layer B.Cu) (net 9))
 (segment (start 174.94999 58.605054) (end 174.309988 57.965052) (width 0.2) (layer B.Cu) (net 9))
 (segment (start 178.55 61.425) (end 178.35 61.225) (width 0.2) (layer F.Cu) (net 13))
 (segment (start 178.55 63.25) (end 178.55 61.425) (width 0.2) (layer F.Cu) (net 13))
 (via (at 178.35 61.225) (size 0.8) (drill 0.4) (layers F.Cu B.Cu) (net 13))
 (via (at 179.05 59.75) (size 0.8) (drill 0.4) (layers F.Cu B.Cu) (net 13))
 (segment (start 176.297451 59.75) (end 179.05 59.75) (width 0.2) (layer F.Cu) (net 13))
 (segment (start 178.35 61.225) (end 178.35 60.45) (width 0.2) (layer B.Cu) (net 13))
 (segment (start 178.35 60.45) (end 179.05 59.75) (width 0.2) (layer B.Cu) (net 13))
 (segment (start 173.173004 65) (end 172.25 65) (width 0.25) (layer F.Cu) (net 16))
 (segment (start 174.398005 63.774999) (end 173.173004 65) (width 0.25) (layer F.Cu) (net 16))
 (segment (start 176.525001 63.774999) (end 174.398005 63.774999) (width 0.25) (layer F.Cu) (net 16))
 (segment (start 177.05 63.25) (end 176.525001 63.774999) (width 0.25) (layer F.Cu) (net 16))
 (segment (start 178.632203 60.559999) (end 179.05 60.977796) (width 0.2) (layer F.Cu) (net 12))
 (segment (start 175.25 61.25) (end 175.940001 60.559999) (width 0.2) (layer F.Cu) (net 12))
 (segment (start 179.05 60.977796) (end 179.05 63.25) (width 0.2) (layer F.Cu) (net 12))
 (segment (start 175.940001 60.559999) (end 178.632203 60.559999) (width 0.2) (layer F.Cu) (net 12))
 (segment (start 187.690002 66.35) (end 187.590002 66.25) (width 0.2) (layer F.Cu) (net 8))
 (via (at 187.590002 66.25) (size 0.8) (drill 0.4) (layers F.Cu B.Cu) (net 8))
 (segment (start 189.3 66.35) (end 187.690002 66.35) (width 0.2) (layer F.Cu) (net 8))
 (via (at 181 62) (size 0.8) (drill 0.4) (layers F.Cu B.Cu) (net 8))
 (segment (start 181.05 62.05) (end 181 62) (width 0.2) (layer F.Cu) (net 8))
 (segment (start 181.05 63.25) (end 181.05 62.05) (width 0.2) (layer F.Cu) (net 8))
 (segment (start 186.9 66.940002) (end 187.190003 66.649999) (width 0.2) (layer B.Cu) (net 8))
 (segment (start 181 62) (end 181 63.747204) (width 0.2) (layer B.Cu) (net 8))
 (segment (start 181 63.747204) (end 184.192798 66.940002) (width 0.2) (layer B.Cu) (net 8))
 (segment (start 184.192798 66.940002) (end 186.9 66.940002) (width 0.2) (layer B.Cu) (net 8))
 (segment (start 187.190003 66.649999) (end 187.590002 66.25) (width 0.2) (layer B.Cu) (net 8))
 (via (at 180.702746 61.108236) (size 0.8) (drill 0.4) (layers F.Cu B.Cu) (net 10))
 (segment (start 180.702746 61.156207) (end 180.702746 61.108236) (width 0.2) (layer F.Cu) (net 10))
 (segment (start 180.05 61.808953) (end 180.702746 61.156207) (width 0.2) (layer F.Cu) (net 10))
 (segment (start 180.05 63.25) (end 180.05 61.808953) (width 0.2) (layer F.Cu) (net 10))
 (segment (start 181.450983 60.359999) (end 183.807201 60.359999) (width 0.2) (layer B.Cu) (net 10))
 (segment (start 180.702746 61.108236) (end 181.450983 60.359999) (width 0.2) (layer B.Cu) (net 10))
 (segment (start 185.95 63.55) (end 185.899999 63.499999) (width 0.2) (layer F.Cu) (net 10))
 (segment (start 189.35 63.55) (end 185.95 63.55) (width 0.2) (layer F.Cu) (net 10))
 (segment (start 185.5 62.052798) (end 185.5 63.1) (width 0.2) (layer B.Cu) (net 10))
 (segment (start 183.807201 60.359999) (end 185.5 62.052798) (width 0.2) (layer B.Cu) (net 10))
 (via (at 185.5 63.1) (size 0.8) (drill 0.4) (layers F.Cu B.Cu) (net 10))
 (segment (start 185.899999 63.499999) (end 185.5 63.1) (width 0.2) (layer F.Cu) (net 10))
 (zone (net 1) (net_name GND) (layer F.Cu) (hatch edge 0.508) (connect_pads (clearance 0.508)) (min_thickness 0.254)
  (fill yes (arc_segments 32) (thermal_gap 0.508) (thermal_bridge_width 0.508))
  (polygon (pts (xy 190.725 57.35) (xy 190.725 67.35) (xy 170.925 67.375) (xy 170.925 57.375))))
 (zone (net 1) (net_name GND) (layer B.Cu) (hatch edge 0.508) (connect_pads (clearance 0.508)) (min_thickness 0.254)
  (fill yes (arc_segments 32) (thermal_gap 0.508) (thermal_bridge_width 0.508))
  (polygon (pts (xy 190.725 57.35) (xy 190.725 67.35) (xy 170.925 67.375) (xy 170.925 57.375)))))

